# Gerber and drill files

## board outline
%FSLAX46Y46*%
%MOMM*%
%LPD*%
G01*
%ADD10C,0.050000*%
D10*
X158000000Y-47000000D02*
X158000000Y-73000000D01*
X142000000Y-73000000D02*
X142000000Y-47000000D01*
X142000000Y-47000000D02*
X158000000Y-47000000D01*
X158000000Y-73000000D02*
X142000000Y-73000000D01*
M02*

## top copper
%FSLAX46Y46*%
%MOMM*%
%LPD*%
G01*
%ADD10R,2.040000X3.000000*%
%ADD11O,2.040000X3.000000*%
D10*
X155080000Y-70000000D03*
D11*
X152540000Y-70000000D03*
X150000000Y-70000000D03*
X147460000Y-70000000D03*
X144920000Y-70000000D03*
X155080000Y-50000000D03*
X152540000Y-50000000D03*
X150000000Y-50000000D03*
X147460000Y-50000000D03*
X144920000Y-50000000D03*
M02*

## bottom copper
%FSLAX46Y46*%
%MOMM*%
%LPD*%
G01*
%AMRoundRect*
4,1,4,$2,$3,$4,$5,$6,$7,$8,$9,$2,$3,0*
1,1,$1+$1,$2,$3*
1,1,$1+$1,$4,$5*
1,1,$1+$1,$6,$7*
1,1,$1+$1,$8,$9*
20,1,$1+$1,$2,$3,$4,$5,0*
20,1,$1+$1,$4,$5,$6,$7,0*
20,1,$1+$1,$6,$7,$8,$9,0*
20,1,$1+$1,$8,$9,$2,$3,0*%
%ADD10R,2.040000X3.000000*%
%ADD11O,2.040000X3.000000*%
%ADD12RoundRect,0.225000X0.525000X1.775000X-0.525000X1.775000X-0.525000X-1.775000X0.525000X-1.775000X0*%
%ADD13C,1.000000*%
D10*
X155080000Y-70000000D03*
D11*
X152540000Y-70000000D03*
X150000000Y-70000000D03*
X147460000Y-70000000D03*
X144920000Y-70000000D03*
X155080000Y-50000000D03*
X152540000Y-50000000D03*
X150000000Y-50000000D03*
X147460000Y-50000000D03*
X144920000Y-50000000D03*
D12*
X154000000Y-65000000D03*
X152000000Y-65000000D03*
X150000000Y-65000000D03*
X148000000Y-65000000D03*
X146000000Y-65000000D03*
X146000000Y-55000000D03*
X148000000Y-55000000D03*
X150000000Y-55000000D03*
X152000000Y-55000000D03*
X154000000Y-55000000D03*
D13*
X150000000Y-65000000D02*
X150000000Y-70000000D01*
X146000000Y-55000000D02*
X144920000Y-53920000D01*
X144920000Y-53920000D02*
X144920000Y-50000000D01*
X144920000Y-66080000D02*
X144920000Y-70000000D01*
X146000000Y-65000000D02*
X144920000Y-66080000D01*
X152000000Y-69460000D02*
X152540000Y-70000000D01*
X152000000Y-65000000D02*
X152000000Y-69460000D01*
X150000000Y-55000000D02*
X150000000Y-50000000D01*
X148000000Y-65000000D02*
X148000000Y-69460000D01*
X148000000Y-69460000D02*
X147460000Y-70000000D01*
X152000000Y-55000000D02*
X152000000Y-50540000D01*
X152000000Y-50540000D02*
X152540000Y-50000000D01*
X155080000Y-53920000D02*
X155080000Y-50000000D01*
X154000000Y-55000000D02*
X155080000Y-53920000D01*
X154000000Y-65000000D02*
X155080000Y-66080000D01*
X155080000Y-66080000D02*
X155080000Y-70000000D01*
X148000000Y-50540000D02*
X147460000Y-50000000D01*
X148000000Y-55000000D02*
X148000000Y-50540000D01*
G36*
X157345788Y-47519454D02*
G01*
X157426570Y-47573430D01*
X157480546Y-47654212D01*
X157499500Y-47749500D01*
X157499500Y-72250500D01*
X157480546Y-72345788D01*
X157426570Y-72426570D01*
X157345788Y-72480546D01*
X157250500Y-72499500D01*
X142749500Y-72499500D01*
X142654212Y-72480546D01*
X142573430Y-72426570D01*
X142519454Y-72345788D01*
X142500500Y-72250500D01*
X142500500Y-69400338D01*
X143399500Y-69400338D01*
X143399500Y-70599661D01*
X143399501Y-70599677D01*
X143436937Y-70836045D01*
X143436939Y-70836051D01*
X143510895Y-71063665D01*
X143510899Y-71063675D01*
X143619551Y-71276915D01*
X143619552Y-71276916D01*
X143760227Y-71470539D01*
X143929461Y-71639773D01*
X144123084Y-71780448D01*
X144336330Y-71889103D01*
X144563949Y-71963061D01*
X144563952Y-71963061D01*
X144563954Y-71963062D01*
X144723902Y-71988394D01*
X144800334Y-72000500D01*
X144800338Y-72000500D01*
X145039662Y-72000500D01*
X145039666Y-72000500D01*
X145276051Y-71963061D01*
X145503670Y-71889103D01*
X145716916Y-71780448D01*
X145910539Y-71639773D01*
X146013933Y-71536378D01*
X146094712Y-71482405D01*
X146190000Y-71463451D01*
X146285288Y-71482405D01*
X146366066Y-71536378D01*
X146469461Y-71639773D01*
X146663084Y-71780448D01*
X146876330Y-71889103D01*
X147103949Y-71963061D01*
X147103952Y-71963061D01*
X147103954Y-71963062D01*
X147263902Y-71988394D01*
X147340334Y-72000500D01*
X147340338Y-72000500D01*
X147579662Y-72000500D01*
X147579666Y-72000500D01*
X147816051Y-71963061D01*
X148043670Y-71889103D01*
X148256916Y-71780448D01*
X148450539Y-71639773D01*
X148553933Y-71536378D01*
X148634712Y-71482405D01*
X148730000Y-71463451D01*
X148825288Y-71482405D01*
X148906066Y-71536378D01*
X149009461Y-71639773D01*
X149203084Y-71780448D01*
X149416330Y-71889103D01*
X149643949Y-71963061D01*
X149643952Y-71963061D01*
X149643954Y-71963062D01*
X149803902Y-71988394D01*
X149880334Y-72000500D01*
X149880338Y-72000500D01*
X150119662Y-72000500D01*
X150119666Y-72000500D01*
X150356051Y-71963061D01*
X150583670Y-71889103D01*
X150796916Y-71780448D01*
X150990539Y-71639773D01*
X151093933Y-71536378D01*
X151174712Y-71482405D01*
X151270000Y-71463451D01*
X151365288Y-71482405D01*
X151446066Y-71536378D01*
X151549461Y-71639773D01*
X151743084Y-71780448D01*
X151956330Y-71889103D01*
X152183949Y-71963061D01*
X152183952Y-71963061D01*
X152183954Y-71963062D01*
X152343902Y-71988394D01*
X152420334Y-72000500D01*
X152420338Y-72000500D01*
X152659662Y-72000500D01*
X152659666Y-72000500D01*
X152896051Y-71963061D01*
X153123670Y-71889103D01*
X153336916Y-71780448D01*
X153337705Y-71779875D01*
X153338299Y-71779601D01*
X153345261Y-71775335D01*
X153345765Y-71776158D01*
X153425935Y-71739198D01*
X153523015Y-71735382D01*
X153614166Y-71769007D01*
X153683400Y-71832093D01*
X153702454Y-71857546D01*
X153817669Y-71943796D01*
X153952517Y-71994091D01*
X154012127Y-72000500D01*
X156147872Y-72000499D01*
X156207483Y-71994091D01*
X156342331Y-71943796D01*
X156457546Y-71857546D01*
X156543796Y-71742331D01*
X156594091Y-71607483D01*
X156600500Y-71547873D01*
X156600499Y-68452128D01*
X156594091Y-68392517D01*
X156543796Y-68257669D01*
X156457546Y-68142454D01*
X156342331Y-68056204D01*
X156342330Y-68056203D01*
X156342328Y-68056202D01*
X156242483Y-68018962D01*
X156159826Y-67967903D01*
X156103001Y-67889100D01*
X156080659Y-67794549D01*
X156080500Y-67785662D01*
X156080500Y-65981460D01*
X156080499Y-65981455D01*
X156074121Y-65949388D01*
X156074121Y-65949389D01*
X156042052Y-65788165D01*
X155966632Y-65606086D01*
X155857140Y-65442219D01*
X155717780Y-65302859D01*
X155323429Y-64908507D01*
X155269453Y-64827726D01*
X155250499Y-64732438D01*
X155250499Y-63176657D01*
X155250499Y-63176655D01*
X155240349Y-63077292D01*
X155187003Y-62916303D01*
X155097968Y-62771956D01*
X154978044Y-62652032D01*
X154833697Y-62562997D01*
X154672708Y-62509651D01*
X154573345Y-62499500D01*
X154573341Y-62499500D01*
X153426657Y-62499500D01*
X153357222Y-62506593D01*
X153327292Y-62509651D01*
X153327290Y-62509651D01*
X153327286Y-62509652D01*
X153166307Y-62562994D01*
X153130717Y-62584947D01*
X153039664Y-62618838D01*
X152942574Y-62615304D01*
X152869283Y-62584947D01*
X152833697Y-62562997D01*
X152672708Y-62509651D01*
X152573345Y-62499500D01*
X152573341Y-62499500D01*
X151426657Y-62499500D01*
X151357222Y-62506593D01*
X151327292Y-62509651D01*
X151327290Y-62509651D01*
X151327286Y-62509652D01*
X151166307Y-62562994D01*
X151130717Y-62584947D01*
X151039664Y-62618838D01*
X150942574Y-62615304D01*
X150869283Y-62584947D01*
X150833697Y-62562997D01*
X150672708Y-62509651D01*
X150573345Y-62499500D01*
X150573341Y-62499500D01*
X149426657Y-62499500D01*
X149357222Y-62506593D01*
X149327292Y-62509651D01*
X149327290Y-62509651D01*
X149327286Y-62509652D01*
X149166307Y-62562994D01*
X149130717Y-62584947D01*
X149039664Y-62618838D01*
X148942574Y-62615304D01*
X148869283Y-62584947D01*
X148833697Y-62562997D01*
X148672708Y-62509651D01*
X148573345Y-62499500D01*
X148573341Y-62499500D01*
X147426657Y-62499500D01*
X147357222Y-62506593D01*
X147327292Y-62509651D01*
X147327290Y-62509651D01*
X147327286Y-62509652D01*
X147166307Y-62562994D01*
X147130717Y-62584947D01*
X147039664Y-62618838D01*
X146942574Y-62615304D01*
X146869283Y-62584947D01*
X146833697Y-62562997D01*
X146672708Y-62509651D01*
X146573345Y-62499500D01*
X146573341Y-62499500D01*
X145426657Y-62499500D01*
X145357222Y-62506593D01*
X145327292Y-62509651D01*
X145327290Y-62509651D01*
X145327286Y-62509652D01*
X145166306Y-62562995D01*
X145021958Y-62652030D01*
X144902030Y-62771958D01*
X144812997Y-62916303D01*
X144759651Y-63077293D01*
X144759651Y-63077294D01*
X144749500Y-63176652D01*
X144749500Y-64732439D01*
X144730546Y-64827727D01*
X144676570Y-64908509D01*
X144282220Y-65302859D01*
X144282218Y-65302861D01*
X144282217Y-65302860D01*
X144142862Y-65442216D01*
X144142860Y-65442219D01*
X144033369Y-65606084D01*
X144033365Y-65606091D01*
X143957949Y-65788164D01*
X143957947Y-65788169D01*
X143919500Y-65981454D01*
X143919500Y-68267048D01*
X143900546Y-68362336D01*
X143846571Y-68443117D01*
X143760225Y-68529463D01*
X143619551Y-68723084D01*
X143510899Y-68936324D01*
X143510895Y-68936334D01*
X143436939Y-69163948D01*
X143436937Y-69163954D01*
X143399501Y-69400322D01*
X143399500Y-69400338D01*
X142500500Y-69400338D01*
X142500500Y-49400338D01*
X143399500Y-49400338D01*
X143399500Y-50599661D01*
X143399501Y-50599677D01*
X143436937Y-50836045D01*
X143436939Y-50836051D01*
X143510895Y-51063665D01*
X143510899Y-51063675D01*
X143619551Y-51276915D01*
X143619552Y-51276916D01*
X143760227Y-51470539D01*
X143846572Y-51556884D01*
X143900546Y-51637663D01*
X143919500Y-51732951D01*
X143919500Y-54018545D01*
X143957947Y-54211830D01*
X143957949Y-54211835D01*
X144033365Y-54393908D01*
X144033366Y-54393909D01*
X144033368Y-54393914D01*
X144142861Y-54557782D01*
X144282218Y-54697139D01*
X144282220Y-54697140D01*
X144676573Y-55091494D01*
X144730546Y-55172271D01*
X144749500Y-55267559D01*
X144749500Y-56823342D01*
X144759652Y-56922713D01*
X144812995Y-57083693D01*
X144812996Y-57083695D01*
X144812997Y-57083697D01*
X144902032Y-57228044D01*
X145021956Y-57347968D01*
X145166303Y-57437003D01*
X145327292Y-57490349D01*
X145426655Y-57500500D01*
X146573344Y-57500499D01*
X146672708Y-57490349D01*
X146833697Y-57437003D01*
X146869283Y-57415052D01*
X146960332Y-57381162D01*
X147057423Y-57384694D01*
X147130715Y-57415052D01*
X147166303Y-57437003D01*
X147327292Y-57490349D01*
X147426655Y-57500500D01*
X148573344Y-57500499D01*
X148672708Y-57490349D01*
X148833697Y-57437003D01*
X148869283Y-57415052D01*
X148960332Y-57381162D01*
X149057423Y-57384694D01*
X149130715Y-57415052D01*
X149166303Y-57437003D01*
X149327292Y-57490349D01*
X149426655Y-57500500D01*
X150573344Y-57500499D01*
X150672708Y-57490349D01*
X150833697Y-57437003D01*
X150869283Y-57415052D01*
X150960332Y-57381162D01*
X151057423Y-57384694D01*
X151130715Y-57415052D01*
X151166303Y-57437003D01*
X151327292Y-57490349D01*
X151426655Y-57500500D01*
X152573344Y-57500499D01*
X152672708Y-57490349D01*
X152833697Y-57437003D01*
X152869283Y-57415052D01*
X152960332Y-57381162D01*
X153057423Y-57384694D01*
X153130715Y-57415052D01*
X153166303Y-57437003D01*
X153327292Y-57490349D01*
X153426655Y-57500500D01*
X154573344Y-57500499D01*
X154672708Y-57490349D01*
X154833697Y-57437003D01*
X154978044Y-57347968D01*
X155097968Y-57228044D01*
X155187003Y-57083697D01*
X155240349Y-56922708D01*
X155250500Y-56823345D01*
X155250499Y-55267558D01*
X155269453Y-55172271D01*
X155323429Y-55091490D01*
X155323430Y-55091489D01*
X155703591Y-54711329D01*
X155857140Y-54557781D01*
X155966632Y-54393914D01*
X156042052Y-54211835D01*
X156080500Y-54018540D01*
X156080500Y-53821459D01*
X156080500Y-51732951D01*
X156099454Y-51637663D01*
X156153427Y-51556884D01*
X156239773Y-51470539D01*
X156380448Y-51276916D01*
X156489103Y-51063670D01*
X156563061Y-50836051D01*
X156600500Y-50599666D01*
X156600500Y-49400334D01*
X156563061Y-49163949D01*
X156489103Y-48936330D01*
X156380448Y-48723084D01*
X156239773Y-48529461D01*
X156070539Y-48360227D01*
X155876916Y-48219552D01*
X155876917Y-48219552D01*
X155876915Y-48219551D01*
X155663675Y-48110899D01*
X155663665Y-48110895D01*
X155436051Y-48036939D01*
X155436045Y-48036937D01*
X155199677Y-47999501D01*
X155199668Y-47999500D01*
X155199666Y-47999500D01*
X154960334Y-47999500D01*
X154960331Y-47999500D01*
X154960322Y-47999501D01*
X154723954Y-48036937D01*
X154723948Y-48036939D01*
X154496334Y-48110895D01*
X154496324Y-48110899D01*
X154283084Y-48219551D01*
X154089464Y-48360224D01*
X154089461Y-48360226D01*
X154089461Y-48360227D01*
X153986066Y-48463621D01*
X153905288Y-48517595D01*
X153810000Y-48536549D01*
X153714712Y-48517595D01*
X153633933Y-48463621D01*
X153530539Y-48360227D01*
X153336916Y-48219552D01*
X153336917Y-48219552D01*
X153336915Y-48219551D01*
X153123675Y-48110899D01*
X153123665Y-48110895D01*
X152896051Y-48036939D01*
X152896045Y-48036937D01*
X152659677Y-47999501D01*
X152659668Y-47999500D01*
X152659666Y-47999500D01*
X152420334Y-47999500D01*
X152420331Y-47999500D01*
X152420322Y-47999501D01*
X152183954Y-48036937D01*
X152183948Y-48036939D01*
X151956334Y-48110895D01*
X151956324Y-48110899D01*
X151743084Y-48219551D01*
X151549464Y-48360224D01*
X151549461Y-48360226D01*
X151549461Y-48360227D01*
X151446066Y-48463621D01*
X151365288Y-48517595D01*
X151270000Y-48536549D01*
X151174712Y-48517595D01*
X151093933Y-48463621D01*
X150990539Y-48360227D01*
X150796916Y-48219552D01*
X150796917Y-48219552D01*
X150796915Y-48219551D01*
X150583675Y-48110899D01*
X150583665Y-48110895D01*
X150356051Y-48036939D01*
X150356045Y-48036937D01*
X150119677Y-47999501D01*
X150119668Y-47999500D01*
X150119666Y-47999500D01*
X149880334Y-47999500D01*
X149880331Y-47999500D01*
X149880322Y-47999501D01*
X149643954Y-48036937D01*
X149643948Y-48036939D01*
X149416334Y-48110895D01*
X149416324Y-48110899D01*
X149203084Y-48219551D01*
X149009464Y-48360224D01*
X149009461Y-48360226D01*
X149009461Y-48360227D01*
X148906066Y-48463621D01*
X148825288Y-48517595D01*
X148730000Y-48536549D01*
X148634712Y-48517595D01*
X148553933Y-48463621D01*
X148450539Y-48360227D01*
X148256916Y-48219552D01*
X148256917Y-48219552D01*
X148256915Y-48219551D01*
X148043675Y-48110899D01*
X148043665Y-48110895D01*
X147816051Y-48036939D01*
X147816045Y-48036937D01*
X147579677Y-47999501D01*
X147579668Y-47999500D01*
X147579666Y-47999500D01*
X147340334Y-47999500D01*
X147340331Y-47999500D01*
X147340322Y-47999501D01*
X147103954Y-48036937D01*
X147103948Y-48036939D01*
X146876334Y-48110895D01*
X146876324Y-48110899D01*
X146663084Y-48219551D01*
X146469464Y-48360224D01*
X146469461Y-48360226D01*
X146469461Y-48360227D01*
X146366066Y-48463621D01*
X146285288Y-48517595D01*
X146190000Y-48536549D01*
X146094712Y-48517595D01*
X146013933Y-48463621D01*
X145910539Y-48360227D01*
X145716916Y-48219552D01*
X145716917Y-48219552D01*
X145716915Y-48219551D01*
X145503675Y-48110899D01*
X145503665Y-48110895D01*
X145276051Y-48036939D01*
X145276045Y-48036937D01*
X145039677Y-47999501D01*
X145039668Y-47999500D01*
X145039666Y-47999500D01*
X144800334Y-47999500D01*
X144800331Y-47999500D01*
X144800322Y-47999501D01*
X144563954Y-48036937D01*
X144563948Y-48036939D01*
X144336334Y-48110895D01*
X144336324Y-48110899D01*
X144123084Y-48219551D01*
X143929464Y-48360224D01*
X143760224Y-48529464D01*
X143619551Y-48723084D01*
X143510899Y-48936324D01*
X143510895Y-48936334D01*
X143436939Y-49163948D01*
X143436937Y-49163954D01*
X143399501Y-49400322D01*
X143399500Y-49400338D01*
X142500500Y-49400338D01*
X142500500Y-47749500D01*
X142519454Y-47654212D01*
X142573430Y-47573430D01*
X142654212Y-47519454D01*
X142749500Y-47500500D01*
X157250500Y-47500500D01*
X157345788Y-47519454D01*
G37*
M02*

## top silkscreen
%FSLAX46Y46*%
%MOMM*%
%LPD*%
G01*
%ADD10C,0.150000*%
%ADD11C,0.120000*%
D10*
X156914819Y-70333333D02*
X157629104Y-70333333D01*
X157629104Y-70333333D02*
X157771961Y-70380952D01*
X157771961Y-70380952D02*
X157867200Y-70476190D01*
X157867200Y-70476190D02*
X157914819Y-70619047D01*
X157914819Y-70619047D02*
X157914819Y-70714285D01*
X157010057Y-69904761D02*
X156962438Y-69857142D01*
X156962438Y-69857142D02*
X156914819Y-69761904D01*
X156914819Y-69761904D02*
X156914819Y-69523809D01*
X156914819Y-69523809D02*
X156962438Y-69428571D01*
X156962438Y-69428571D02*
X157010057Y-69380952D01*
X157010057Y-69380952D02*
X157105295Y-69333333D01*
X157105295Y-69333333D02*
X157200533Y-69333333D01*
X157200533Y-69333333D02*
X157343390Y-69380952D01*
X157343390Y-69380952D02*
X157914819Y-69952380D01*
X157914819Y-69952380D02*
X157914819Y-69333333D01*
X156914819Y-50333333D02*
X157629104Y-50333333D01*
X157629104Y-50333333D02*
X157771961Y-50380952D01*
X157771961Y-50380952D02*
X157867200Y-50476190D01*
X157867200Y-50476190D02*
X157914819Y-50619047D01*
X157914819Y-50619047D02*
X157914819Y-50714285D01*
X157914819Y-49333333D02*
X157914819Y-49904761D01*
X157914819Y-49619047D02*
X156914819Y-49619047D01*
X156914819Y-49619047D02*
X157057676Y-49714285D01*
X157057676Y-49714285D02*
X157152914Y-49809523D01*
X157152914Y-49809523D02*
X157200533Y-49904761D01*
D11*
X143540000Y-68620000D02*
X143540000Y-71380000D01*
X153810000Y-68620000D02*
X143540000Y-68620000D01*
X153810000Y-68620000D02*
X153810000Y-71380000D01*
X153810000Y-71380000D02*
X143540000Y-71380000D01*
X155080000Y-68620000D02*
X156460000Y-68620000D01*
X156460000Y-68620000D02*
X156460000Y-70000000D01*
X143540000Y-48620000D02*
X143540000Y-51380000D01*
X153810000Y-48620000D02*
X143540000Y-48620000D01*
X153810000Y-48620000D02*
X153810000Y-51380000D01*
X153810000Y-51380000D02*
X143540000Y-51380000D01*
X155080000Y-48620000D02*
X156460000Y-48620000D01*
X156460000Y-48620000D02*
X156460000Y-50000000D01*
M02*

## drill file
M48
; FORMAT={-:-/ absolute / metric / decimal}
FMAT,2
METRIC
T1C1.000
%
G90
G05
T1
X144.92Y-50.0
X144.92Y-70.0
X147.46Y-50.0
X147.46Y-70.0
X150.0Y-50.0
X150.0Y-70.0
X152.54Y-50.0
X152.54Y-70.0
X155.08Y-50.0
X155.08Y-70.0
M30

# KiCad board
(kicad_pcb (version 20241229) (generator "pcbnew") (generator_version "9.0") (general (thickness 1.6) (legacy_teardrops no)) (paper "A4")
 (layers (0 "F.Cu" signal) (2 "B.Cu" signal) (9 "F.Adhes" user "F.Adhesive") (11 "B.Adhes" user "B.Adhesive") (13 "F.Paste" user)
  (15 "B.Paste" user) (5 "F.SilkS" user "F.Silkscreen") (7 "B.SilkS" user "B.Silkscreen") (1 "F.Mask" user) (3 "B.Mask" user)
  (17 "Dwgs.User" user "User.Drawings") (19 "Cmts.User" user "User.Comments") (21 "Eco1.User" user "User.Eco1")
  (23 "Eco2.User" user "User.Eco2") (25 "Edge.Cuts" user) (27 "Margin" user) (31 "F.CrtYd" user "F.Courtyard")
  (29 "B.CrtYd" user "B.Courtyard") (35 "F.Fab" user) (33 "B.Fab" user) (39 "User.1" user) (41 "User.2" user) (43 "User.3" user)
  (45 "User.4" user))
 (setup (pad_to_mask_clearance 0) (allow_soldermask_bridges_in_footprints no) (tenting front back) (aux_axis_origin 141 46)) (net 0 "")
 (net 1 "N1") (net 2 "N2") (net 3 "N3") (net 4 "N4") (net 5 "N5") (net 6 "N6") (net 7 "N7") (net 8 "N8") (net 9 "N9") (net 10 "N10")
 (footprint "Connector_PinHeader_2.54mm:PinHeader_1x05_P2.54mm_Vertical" (layer "F.Cu") (at 155.08 70 -90)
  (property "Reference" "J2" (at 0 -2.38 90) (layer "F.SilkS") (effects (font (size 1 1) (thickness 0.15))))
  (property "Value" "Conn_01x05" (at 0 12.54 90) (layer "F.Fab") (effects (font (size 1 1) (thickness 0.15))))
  (fp_line (start -1.38 11.54) (end 1.38 11.54) (stroke (width 0.12) (type solid)) (layer "F.SilkS"))
  (fp_line (start -1.38 1.27) (end -1.38 11.54) (stroke (width 0.12) (type solid)) (layer "F.SilkS"))
  (fp_line (start -1.38 1.27) (end 1.38 1.27) (stroke (width 0.12) (type solid)) (layer "F.SilkS"))
  (fp_line (start 1.38 1.27) (end 1.38 11.54) (stroke (width 0.12) (type solid)) (layer "F.SilkS"))
  (fp_line (start -1.38 0) (end -1.38 -1.38) (stroke (width 0.12) (type solid)) (layer "F.SilkS"))
  (fp_line (start -1.38 -1.38) (end 0 -1.38) (stroke (width 0.12) (type solid)) (layer "F.SilkS"))
  (pad "1" thru_hole rect (at 0 0 270) (size 3 2.04) (drill 1) (layers "*.Cu" "*.Mask") (remove_unused_layers no) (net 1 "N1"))
  (pad "2" thru_hole oval (at 0 2.54 270) (size 3 2.04) (drill 1) (layers "*.Cu" "*.Mask") (remove_unused_layers no) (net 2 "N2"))
  (pad "3" thru_hole oval (at 0 5.08 270) (size 3 2.04) (drill 1) (layers "*.Cu" "*.Mask") (remove_unused_layers no) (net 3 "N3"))
  (pad "4" thru_hole oval (at 0 7.62 270) (size 3 2.04) (drill 1) (layers "*.Cu" "*.Mask") (remove_unused_layers no) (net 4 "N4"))
  (pad "5" thru_hole oval (at 0 10.16 270) (size 3 2.04) (drill 1) (layers "*.Cu" "*.Mask") (remove_unused_layers no) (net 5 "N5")))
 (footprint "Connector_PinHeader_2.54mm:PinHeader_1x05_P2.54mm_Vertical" (layer "F.Cu") (at 155.08 50 -90)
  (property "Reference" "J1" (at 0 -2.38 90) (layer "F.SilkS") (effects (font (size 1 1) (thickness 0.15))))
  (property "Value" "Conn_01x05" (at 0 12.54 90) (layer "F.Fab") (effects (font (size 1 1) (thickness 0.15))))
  (fp_line (start -1.38 11.54) (end 1.38 11.54) (stroke (width 0.12) (type solid)) (layer "F.SilkS"))
  (fp_line (start -1.38 1.27) (end -1.38 11.54) (stroke (width 0.12) (type solid)) (layer "F.SilkS"))
  (fp_line (start -1.38 1.27) (end 1.38 1.27) (stroke (width 0.12) (type solid)) (layer "F.SilkS"))
  (fp_line (start 1.38 1.27) (end 1.38 11.54) (stroke (width 0.12) (type solid)) (layer "F.SilkS"))
  (fp_line (start -1.38 0) (end -1.38 -1.38) (stroke (width 0.12) (type solid)) (layer "F.SilkS"))
  (fp_line (start -1.38 -1.38) (end 0 -1.38) (stroke (width 0.12) (type solid)) (layer "F.SilkS"))
  (pad "1" thru_hole oval (at 0 0 270) (size 3 2.04) (drill 1) (layers "*.Cu" "*.Mask") (remove_unused_layers no) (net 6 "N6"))
  (pad "2" thru_hole oval (at 0 2.54 270) (size 3 2.04) (drill 1) (layers "*.Cu" "*.Mask") (remove_unused_layers no) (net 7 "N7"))
  (pad "3" thru_hole oval (at 0 5.08 270) (size 3 2.04) (drill 1) (layers "*.Cu" "*.Mask") (remove_unused_layers no) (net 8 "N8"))
  (pad "4" thru_hole oval (at 0 7.62 270) (size 3 2.04) (drill 1) (layers "*.Cu" "*.Mask") (remove_unused_layers no) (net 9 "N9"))
  (pad "5" thru_hole oval (at 0 10.16 270) (size 3 2.04) (drill 1) (layers "*.Cu" "*.Mask") (remove_unused_layers no) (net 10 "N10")))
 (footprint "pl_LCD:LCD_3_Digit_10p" (layer "B.Cu") (at 150 60 180)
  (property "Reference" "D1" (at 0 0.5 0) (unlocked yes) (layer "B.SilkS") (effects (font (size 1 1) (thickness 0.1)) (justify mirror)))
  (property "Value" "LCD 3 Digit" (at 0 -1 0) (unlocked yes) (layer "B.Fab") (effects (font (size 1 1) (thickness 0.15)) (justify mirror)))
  (pad "1" smd roundrect (at -4 -5 180) (size 1.5 4) (layers "B.Cu" "B.Mask" "B.Paste") (roundrect_rratio 0.15) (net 1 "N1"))
  (pad "2" smd roundrect (at -2 -5 180) (size 1.5 4) (layers "B.Cu" "B.Mask" "B.Paste") (roundrect_rratio 0.15) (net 2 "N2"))
  (pad "3" smd roundrect (at 0 -5 180) (size 1.5 4) (layers "B.Cu" "B.Mask" "B.Paste") (roundrect_rratio 0.15) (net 3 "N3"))
  (pad "4" smd roundrect (at 2 -5 180) (size 1.5 4) (layers "B.Cu" "B.Mask" "B.Paste") (roundrect_rratio 0.15) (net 4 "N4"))
  (pad "5" smd roundrect (at 4 -5 180) (size 1.5 4) (layers "B.Cu" "B.Mask" "B.Paste") (roundrect_rratio 0.15) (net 5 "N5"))
  (pad "6" smd roundrect (at 4 5 180) (size 1.5 4) (layers "B.Cu" "B.Mask" "B.Paste") (roundrect_rratio 0.15) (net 10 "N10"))
  (pad "7" smd roundrect (at 2 5 180) (size 1.5 4) (layers "B.Cu" "B.Mask" "B.Paste") (roundrect_rratio 0.15) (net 9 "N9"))
  (pad "8" smd roundrect (at 0 5 180) (size 1.5 4) (layers "B.Cu" "B.Mask" "B.Paste") (roundrect_rratio 0.15) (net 8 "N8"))
  (pad "9" smd roundrect (at -2 5 180) (size 1.5 4) (layers "B.Cu" "B.Mask" "B.Paste") (roundrect_rratio 0.15) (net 7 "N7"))
  (pad "10" smd roundrect (at -4 5 180) (size 1.5 4) (layers "B.Cu" "B.Mask" "B.Paste") (roundrect_rratio 0.15) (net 6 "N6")))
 (gr_line (start 158 47) (end 158 73) (stroke (width 0.05) (type default)) (layer "Edge.Cuts"))
 (gr_line (start 142 73) (end 142 47) (stroke (width 0.05) (type default)) (layer "Edge.Cuts"))
 (gr_line (start 142 47) (end 158 47) (stroke (width 0.05) (type default)) (layer "Edge.Cuts"))
 (gr_line (start 158 73) (end 142 73) (stroke (width 0.05) (type default)) (layer "Edge.Cuts"))
 (segment (start 150 65) (end 150 70) (width 1) (layer "B.Cu") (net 3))
 (segment (start 146 55) (end 144.92 53.92) (width 1) (layer "B.Cu") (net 10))
 (segment (start 144.92 53.92) (end 144.92 50) (width 1) (layer "B.Cu") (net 10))
 (segment (start 144.92 66.08) (end 144.92 70) (width 1) (layer "B.Cu") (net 5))
 (segment (start 146 65) (end 144.92 66.08) (width 1) (layer "B.Cu") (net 5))
 (segment (start 152 69.46) (end 152.54 70) (width 1) (layer "B.Cu") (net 2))
 (segment (start 152 65) (end 152 69.46) (width 1) (layer "B.Cu") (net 2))
 (segment (start 150 55) (end 150 50) (width 1) (layer "B.Cu") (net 8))
 (segment (start 148 65) (end 148 69.46) (width 1) (layer "B.Cu") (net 4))
 (segment (start 148 69.46) (end 147.46 70) (width 1) (layer "B.Cu") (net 4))
 (segment (start 152 55) (end 152 50.54) (width 1) (layer "B.Cu") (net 7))
 (segment (start 152 50.54) (end 152.54 50) (width 1) (layer "B.Cu") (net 7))
 (segment (start 155.08 53.92) (end 155.08 50) (width 1) (layer "B.Cu") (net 6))
 (segment (start 154 55) (end 155.08 53.92) (width 1) (layer "B.Cu") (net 6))
 (segment (start 154 65) (end 155.08 66.08) (width 1) (layer "B.Cu") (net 1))
 (segment (start 155.08 66.08) (end 155.08 70) (width 1) (layer "B.Cu") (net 1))
 (segment (start 148 50.54) (end 147.46 50) (width 1) (layer "B.Cu") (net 9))
 (segment (start 148 55) (end 148 50.54) (width 1) (layer "B.Cu") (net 9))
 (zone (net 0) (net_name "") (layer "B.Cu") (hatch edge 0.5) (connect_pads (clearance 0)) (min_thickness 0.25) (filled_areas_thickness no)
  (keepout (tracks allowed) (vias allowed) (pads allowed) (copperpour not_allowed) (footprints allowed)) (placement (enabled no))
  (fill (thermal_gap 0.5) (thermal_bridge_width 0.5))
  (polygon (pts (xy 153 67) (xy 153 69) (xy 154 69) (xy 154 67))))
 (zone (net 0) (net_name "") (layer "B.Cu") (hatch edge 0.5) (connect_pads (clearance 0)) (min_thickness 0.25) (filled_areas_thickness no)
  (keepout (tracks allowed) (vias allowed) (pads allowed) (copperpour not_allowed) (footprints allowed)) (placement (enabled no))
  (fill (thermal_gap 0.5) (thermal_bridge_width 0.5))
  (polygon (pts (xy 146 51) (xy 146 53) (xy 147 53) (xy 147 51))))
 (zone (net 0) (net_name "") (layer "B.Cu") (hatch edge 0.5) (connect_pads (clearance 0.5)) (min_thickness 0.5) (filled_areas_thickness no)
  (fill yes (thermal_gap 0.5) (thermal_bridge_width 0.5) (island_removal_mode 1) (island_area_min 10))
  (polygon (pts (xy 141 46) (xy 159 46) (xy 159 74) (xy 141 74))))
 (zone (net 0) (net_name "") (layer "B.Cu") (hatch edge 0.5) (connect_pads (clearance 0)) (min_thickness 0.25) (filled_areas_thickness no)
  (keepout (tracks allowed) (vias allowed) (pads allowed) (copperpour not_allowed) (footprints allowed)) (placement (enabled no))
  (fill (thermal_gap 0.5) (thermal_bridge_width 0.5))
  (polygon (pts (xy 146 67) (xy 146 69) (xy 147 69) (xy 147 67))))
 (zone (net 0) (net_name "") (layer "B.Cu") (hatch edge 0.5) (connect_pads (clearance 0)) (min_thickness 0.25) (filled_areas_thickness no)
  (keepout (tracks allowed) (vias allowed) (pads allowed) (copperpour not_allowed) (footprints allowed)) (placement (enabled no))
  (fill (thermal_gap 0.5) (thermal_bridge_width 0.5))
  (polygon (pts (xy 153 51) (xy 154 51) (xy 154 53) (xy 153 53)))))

